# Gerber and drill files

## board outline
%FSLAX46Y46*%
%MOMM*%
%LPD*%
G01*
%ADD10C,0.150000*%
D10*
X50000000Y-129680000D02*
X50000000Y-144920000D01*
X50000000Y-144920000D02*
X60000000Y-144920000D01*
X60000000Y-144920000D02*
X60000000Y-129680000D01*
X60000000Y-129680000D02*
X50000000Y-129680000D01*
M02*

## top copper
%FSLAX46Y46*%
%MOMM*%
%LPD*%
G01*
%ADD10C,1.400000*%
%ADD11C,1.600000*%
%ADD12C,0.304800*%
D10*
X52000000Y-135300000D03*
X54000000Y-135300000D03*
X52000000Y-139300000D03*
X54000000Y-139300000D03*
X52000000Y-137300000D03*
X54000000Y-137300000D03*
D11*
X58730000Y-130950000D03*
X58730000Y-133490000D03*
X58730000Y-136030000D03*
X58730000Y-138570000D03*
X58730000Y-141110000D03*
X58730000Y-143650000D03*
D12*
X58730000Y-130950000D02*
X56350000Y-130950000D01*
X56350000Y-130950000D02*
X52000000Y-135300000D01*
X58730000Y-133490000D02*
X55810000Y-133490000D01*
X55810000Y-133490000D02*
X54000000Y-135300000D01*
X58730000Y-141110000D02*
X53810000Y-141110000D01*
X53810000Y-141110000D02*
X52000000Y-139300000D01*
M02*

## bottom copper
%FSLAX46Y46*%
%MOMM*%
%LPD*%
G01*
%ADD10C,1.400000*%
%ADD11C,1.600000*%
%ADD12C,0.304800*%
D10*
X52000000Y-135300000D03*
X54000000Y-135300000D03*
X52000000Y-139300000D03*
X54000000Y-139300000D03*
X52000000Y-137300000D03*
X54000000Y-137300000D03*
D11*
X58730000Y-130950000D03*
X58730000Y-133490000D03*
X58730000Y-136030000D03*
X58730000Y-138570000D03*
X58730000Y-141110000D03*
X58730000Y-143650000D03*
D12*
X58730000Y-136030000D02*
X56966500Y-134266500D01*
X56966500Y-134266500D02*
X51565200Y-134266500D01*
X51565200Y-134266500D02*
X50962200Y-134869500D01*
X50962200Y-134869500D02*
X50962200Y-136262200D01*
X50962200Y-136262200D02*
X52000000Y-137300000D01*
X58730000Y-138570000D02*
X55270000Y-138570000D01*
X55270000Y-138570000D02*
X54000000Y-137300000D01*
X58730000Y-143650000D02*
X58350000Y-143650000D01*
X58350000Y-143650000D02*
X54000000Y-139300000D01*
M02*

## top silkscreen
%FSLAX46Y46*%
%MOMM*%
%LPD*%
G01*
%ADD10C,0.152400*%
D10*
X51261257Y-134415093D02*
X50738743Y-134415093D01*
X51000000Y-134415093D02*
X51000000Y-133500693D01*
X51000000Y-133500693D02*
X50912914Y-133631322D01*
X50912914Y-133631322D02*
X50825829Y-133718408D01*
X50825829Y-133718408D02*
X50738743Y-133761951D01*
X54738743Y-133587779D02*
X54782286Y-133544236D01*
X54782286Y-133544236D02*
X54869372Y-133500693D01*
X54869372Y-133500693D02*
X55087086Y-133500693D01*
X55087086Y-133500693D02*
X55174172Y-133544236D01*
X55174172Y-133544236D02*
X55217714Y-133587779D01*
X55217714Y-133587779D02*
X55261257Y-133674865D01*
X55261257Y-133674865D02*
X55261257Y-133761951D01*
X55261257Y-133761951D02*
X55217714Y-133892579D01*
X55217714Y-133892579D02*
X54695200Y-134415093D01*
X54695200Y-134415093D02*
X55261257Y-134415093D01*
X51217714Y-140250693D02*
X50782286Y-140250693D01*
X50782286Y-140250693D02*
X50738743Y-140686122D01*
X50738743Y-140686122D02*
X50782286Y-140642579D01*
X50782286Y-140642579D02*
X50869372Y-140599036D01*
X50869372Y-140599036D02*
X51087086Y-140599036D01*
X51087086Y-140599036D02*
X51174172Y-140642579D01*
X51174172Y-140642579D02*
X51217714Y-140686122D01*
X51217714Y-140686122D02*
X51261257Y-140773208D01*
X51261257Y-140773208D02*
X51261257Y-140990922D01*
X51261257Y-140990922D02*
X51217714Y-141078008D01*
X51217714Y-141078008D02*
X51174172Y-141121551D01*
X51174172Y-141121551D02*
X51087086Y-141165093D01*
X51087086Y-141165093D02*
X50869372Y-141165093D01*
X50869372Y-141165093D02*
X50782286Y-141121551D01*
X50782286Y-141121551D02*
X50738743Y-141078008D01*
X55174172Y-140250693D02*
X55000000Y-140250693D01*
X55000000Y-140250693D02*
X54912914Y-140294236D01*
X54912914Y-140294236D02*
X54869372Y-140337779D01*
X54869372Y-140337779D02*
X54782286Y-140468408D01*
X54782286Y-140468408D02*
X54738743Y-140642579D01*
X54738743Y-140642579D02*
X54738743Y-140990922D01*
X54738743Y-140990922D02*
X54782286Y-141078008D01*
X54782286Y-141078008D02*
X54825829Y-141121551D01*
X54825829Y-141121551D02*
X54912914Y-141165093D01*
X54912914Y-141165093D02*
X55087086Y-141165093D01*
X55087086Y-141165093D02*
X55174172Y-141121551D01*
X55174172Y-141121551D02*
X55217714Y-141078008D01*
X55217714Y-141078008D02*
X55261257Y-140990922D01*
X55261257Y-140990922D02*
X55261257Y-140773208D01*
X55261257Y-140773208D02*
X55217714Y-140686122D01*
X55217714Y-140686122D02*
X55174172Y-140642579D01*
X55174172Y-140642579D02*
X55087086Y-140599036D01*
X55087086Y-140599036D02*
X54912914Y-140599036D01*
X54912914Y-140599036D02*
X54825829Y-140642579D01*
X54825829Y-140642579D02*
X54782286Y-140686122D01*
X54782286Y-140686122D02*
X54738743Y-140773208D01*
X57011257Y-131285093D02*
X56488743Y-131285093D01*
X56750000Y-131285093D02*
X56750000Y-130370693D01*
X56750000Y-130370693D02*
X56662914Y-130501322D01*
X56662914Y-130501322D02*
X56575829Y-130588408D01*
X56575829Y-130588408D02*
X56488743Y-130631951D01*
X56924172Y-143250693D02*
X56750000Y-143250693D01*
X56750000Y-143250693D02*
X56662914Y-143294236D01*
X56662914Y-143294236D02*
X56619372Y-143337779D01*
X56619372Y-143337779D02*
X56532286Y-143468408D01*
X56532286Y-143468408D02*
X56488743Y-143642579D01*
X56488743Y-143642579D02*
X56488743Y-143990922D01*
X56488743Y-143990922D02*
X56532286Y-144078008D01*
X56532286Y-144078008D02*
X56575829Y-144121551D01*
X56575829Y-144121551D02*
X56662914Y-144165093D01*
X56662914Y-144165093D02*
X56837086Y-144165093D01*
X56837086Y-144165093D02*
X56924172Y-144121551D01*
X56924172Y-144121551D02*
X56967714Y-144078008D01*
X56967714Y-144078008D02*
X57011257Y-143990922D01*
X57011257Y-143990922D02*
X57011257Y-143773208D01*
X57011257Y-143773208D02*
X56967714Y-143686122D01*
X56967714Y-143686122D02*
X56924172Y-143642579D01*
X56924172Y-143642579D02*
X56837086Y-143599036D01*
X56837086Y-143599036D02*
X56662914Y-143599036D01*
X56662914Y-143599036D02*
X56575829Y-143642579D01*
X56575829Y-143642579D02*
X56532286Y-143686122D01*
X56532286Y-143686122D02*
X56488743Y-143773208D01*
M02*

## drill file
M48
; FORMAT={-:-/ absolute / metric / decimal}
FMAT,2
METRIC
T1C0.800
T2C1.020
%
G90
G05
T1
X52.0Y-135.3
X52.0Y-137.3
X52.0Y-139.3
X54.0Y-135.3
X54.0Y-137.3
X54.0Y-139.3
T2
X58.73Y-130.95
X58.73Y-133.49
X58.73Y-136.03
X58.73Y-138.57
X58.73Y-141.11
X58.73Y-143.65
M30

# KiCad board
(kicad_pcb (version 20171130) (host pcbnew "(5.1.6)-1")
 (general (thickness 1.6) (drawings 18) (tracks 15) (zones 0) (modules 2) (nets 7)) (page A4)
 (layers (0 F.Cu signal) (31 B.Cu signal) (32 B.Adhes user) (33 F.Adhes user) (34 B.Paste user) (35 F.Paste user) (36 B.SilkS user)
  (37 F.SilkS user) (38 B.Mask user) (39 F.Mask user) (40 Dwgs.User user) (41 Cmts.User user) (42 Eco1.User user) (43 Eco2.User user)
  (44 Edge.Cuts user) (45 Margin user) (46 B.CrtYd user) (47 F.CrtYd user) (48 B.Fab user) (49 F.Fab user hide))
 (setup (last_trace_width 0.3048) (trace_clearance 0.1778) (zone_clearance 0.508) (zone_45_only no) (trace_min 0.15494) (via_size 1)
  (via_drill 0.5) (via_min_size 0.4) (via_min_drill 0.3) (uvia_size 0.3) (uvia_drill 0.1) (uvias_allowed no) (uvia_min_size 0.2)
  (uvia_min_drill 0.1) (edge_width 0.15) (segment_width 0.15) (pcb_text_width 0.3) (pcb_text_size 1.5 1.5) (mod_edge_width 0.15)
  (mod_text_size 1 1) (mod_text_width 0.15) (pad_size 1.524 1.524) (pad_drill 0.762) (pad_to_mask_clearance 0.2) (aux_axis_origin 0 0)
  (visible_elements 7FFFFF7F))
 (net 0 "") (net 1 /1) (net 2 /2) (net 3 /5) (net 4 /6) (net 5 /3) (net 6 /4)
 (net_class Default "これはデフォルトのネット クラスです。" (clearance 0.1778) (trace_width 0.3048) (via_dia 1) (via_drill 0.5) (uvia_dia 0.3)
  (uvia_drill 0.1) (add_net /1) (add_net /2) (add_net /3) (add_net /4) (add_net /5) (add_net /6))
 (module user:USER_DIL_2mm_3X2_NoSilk (layer F.Cu) (at 53 137.3)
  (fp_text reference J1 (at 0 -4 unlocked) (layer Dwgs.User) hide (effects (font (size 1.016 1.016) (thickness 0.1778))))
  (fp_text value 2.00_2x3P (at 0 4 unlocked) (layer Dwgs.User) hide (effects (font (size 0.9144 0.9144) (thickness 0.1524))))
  (pad 1 thru_hole circle (at -1 -2) (size 1.4 1.4) (drill 0.8) (layers *.Cu *.Mask) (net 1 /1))
  (pad 2 thru_hole circle (at 1 -2) (size 1.4 1.4) (drill 0.8) (layers *.Cu *.Mask) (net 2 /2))
  (pad 5 thru_hole circle (at -1 2) (size 1.4 1.4) (drill 0.8) (layers *.Cu *.Mask) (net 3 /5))
  (pad 6 thru_hole circle (at 1 2) (size 1.4 1.4) (drill 0.8) (layers *.Cu *.Mask) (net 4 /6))
  (pad 3 thru_hole circle (at -1 0) (size 1.4 1.4) (drill 0.8) (layers *.Cu *.Mask) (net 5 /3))
  (pad 4 thru_hole circle (at 1 0) (size 1.4 1.4) (drill 0.8) (layers *.Cu *.Mask) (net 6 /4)))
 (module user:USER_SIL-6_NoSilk (layer F.Cu) (at 58.73 137.3 270)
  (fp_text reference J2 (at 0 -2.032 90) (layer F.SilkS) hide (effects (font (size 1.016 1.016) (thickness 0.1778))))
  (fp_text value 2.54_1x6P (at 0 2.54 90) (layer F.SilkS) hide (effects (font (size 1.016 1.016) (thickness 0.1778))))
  (pad 1 thru_hole circle (at -6.35 0 270) (size 1.6 1.6) (drill 1.02) (layers *.Cu *.Mask) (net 1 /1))
  (pad 2 thru_hole circle (at -3.81 0 270) (size 1.6 1.6) (drill 1.02) (layers *.Cu *.Mask) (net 2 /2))
  (pad 3 thru_hole circle (at -1.27 0 270) (size 1.6 1.6) (drill 1.02) (layers *.Cu *.Mask) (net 5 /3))
  (pad 4 thru_hole circle (at 1.27 0 270) (size 1.6 1.6) (drill 1.02) (layers *.Cu *.Mask) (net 6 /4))
  (pad 5 thru_hole circle (at 3.81 0 270) (size 1.6 1.6) (drill 1.02) (layers *.Cu *.Mask) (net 3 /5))
  (pad 6 thru_hole circle (at 6.35 0 270) (size 1.6 1.6) (drill 1.02) (layers *.Cu *.Mask) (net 4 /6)))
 (gr_line (start 50 129.68) (end 50 144.92) (angle 90) (layer Edge.Cuts) (width 0.15))
 (gr_line (start 50 144.92) (end 60 144.92) (angle 90) (layer Edge.Cuts) (width 0.15))
 (gr_line (start 60 144.92) (end 60 129.68) (angle 90) (layer Edge.Cuts) (width 0.15))
 (gr_line (start 60 129.68) (end 50 129.68) (angle 90) (layer Edge.Cuts) (width 0.15))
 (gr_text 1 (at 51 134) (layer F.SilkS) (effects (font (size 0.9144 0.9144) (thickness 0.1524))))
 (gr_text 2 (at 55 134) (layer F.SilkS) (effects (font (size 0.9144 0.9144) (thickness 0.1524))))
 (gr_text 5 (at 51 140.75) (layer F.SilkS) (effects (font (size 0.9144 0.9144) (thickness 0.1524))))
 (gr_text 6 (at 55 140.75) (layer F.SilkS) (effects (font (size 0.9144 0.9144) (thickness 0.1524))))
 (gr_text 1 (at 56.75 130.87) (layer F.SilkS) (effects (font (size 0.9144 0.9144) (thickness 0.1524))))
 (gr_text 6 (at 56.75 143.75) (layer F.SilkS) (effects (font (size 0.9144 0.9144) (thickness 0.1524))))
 (segment (start 58.73 130.95) (end 56.35 130.95) (width 0.3048) (layer F.Cu) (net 1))
 (segment (start 56.35 130.95) (end 52 135.3) (width 0.3048) (layer F.Cu) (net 1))
 (segment (start 58.73 133.49) (end 55.81 133.49) (width 0.3048) (layer F.Cu) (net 2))
 (segment (start 55.81 133.49) (end 54 135.3) (width 0.3048) (layer F.Cu) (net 2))
 (segment (start 58.73 136.03) (end 56.9665 134.2665) (width 0.3048) (layer B.Cu) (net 5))
 (segment (start 56.9665 134.2665) (end 51.5652 134.2665) (width 0.3048) (layer B.Cu) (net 5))
 (segment (start 51.5652 134.2665) (end 50.9622 134.8695) (width 0.3048) (layer B.Cu) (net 5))
 (segment (start 50.9622 134.8695) (end 50.9622 136.2622) (width 0.3048) (layer B.Cu) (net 5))
 (segment (start 50.9622 136.2622) (end 52 137.3) (width 0.3048) (layer B.Cu) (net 5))
 (segment (start 58.73 138.57) (end 55.27 138.57) (width 0.3048) (layer B.Cu) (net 6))
 (segment (start 55.27 138.57) (end 54 137.3) (width 0.3048) (layer B.Cu) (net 6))
 (segment (start 58.73 141.11) (end 53.81 141.11) (width 0.3048) (layer F.Cu) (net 3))
 (segment (start 53.81 141.11) (end 52 139.3) (width 0.3048) (layer F.Cu) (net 3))
 (segment (start 58.73 143.65) (end 58.35 143.65) (width 0.3048) (layer B.Cu) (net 4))
 (segment (start 58.35 143.65) (end 54 139.3) (width 0.3048) (layer B.Cu) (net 4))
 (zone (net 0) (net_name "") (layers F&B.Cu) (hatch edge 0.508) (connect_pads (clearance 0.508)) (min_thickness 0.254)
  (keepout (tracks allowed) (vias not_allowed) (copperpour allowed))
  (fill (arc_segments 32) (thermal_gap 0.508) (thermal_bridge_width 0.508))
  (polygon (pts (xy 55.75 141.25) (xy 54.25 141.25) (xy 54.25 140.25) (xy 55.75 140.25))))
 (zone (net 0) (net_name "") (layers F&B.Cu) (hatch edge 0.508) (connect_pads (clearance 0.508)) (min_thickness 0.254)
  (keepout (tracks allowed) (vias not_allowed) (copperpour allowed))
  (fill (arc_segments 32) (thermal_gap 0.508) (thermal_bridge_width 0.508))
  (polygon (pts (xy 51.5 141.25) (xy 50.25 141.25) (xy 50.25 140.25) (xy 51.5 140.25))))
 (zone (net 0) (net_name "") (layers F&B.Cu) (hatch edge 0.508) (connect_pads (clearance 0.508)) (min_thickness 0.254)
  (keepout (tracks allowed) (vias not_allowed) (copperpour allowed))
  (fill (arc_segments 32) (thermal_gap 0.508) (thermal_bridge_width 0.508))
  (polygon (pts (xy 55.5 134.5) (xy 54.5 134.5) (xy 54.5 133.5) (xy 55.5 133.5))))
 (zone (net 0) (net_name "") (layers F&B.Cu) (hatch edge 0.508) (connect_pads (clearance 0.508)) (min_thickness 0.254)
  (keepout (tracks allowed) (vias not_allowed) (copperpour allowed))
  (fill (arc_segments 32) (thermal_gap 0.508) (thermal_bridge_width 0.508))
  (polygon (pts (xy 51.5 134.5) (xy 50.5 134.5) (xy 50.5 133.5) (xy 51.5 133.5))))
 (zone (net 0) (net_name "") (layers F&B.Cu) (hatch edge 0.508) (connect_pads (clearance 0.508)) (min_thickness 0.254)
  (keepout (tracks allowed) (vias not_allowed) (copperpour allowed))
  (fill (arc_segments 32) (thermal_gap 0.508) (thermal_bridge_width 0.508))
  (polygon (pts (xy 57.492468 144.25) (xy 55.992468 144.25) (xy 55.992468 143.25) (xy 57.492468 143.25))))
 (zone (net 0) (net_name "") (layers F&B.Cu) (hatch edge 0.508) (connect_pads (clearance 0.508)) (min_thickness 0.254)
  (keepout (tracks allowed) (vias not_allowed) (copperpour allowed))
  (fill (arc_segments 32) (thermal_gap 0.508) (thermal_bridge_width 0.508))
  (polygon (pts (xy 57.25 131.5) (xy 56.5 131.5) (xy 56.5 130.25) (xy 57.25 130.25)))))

